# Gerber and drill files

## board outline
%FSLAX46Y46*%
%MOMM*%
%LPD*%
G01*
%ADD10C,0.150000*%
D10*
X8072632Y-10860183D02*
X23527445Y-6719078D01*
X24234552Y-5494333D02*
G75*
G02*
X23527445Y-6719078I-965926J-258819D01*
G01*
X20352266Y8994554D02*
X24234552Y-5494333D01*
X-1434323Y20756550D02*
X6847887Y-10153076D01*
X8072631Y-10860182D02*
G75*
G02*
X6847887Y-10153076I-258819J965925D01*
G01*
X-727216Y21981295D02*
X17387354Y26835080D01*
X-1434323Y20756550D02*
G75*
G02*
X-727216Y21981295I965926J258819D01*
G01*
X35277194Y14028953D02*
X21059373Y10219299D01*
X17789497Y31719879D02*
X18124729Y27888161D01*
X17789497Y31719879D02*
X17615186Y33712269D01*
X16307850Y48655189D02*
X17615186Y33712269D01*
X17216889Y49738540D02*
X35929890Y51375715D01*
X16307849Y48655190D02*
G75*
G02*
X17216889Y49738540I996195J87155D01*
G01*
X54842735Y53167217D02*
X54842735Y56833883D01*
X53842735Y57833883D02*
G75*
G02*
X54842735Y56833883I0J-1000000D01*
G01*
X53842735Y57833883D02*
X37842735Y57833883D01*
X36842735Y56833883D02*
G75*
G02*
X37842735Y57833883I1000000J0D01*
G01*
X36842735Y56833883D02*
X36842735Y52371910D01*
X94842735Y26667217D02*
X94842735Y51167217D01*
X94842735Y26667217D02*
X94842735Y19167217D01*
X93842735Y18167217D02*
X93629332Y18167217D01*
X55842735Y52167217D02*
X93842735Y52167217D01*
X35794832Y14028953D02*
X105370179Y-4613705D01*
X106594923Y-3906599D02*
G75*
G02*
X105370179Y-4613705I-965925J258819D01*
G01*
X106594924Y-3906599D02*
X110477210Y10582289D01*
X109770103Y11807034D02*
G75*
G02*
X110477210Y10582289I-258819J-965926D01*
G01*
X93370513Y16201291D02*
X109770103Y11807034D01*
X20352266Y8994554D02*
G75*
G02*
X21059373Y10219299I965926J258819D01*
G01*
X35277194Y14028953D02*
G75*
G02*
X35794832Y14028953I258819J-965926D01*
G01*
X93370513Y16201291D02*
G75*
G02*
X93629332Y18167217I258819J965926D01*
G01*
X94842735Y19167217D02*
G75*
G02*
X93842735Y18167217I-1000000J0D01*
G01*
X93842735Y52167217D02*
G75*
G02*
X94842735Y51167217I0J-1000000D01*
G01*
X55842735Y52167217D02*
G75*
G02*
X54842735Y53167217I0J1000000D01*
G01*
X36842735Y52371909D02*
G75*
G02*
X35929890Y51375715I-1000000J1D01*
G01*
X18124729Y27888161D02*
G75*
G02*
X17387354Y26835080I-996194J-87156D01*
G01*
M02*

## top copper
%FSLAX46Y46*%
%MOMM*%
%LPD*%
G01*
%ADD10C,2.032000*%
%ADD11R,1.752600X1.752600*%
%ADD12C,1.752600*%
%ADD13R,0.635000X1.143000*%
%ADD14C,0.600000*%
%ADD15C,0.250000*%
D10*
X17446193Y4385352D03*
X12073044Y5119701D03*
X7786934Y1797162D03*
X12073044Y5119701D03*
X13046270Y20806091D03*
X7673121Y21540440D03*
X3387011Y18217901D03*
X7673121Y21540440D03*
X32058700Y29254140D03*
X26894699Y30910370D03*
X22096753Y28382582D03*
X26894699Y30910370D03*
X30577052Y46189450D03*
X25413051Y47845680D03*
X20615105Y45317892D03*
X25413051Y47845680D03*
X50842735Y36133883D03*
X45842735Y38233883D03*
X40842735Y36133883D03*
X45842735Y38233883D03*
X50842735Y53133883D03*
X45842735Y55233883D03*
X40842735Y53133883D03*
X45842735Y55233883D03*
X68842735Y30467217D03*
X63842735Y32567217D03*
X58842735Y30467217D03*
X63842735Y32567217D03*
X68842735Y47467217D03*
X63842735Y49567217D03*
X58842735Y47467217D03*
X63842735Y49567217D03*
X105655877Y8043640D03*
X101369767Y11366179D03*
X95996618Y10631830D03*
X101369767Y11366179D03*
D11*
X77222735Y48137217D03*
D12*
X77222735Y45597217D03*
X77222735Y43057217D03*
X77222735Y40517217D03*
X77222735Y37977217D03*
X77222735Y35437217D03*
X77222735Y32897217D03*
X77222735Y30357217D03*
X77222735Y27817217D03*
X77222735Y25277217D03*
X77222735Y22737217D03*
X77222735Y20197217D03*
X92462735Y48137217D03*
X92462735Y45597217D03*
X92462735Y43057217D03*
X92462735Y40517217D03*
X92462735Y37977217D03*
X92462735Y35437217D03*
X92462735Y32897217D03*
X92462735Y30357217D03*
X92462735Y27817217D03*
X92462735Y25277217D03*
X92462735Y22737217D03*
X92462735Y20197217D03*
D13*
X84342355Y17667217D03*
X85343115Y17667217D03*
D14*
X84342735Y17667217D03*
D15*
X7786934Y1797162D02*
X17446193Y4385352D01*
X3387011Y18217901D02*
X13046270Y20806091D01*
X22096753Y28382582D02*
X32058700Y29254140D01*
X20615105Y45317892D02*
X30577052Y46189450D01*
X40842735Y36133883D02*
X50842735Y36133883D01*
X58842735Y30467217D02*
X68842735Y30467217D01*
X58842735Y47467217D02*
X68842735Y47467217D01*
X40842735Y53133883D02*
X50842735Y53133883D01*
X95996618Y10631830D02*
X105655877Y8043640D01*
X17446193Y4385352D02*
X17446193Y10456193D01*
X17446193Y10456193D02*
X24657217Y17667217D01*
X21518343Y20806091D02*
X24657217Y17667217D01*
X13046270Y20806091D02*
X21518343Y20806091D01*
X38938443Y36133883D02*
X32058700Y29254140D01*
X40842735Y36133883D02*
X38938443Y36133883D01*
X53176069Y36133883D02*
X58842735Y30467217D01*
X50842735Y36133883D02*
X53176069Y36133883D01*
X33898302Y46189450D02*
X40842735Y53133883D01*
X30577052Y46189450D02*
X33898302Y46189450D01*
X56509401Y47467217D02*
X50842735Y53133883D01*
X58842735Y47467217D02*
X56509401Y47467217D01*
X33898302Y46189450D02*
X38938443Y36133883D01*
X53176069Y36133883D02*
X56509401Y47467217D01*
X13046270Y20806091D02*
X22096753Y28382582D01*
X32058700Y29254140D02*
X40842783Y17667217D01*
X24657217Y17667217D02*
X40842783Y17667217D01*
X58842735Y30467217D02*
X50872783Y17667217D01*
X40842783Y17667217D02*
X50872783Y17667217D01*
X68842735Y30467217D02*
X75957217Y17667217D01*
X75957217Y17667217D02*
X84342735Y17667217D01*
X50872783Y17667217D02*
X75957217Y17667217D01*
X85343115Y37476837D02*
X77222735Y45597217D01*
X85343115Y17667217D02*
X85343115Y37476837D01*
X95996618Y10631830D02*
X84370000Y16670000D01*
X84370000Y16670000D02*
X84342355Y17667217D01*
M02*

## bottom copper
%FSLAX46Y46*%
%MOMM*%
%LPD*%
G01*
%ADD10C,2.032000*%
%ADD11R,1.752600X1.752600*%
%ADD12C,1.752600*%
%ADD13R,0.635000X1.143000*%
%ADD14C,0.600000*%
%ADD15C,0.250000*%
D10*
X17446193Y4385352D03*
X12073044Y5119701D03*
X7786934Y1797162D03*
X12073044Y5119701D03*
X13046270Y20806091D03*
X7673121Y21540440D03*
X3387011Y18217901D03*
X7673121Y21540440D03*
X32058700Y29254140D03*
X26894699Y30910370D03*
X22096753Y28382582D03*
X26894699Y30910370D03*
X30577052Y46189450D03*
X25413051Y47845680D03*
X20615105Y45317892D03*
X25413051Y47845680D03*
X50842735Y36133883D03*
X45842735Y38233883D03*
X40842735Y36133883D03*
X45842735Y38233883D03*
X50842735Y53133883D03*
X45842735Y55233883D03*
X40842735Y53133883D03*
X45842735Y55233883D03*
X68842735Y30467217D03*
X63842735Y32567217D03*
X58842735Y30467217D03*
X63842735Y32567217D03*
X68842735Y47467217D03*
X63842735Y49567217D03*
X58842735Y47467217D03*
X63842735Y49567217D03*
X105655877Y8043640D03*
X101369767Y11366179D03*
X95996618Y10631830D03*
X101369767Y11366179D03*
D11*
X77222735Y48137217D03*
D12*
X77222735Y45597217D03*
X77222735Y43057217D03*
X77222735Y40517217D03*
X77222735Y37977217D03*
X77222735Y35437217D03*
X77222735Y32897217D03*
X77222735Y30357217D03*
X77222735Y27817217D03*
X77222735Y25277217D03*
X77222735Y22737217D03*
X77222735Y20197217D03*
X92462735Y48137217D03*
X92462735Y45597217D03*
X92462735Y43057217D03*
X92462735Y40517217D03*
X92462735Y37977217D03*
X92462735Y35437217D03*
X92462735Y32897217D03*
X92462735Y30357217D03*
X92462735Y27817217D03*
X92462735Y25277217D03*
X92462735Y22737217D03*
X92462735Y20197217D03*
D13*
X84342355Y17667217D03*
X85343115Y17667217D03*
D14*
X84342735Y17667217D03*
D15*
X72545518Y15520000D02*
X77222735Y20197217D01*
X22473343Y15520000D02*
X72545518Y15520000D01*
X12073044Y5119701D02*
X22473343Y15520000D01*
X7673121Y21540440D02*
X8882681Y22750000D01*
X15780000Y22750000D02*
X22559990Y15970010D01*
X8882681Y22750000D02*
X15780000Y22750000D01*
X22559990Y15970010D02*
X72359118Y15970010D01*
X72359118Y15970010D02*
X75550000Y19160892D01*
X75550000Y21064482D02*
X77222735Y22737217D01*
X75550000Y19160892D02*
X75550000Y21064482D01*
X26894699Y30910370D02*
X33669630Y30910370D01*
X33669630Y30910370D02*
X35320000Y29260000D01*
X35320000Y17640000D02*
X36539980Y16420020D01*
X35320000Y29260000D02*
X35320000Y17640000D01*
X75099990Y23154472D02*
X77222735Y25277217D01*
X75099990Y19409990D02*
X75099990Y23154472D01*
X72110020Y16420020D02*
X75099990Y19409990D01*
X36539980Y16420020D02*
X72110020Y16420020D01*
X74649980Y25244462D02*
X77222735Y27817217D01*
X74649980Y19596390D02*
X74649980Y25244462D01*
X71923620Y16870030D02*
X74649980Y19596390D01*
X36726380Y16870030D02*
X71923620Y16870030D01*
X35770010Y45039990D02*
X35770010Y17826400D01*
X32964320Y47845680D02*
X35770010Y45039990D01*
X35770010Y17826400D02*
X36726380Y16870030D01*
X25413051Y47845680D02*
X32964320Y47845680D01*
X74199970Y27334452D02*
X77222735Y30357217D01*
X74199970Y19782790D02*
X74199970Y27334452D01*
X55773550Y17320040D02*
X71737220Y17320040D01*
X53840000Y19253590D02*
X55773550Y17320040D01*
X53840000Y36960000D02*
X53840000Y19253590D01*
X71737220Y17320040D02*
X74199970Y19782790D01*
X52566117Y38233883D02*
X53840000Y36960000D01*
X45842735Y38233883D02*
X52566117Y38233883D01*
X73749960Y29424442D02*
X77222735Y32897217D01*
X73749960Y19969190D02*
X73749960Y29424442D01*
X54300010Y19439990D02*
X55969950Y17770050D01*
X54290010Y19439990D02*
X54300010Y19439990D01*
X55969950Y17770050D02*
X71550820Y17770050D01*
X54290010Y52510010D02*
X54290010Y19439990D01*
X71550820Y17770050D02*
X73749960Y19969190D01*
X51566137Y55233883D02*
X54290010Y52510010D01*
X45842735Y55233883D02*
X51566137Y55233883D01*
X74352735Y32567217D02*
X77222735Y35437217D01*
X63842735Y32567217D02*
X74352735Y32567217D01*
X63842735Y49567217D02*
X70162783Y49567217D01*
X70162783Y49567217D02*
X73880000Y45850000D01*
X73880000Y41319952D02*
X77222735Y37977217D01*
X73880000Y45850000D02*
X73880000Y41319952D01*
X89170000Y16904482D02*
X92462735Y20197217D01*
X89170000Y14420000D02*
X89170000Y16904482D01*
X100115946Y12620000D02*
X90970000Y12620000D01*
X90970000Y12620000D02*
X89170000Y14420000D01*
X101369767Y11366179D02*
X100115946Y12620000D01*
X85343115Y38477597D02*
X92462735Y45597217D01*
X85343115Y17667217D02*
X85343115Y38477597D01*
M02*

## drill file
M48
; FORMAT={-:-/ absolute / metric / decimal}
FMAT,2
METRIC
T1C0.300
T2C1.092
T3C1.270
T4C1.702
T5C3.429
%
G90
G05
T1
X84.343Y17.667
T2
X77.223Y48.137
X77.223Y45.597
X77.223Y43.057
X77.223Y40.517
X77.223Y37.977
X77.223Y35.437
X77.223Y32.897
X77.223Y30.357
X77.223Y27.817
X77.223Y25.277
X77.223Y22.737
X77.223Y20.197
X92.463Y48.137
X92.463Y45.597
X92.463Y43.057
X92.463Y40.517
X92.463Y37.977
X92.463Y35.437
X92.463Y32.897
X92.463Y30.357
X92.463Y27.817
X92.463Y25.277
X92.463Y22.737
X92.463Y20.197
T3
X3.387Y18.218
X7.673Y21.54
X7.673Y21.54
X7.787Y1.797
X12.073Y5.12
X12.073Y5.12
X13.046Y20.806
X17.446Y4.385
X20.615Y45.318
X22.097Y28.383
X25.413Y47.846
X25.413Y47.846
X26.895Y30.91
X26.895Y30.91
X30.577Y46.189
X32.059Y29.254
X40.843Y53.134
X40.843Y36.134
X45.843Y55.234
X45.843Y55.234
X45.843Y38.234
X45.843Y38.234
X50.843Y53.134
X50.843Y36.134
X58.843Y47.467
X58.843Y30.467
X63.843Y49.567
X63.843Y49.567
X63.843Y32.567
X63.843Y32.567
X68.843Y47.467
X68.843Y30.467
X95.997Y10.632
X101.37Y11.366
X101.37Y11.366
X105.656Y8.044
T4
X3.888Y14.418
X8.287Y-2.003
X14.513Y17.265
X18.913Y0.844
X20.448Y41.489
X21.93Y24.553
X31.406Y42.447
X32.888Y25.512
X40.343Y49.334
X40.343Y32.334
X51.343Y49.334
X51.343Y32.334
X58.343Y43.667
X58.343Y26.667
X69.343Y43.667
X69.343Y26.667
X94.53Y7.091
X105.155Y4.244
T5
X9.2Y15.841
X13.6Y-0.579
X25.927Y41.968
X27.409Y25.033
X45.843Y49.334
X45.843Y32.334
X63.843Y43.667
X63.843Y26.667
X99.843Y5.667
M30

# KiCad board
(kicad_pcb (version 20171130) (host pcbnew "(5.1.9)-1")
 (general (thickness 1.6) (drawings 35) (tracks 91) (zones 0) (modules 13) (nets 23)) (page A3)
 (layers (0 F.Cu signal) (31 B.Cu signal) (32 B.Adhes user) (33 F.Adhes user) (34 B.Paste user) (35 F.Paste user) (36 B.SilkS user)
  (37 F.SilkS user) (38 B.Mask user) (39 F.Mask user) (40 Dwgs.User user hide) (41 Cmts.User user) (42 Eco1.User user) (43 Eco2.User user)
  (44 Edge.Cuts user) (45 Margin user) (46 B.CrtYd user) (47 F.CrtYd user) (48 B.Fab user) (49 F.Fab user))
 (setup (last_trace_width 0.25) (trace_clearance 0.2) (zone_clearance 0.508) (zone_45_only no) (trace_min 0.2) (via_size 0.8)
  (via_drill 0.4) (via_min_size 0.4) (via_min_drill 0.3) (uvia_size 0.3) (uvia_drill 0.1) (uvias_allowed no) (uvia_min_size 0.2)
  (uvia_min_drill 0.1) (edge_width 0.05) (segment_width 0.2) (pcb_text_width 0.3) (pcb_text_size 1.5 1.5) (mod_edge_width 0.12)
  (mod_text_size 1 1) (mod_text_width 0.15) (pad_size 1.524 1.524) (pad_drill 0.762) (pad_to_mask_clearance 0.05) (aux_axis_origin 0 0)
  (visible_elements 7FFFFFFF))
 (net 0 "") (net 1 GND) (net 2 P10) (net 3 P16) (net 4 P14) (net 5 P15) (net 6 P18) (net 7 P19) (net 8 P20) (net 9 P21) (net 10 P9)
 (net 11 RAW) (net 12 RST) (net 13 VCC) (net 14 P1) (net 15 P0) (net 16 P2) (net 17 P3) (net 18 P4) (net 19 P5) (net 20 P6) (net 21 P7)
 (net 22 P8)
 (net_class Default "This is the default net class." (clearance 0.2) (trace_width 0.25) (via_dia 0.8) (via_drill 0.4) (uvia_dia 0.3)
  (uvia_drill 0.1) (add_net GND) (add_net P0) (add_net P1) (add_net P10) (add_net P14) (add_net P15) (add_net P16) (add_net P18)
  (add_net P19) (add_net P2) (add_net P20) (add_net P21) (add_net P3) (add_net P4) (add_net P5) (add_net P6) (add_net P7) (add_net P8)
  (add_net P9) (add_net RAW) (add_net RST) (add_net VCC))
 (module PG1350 (layer F.Cu) (at 13.600076 0.579261 15)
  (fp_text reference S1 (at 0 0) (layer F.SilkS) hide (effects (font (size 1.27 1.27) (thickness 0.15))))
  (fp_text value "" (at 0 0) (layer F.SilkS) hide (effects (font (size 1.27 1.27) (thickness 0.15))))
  (pad "" np_thru_hole circle (at 0 0) (size 3.429 3.429) (drill 3.429) (layers *.Cu *.Mask))
  (pad "" np_thru_hole circle (at 5.5 0) (size 1.7018 1.7018) (drill 1.7018) (layers *.Cu *.Mask))
  (pad "" np_thru_hole circle (at -5.5 0) (size 1.7018 1.7018) (drill 1.7018) (layers *.Cu *.Mask))
  (pad 1 thru_hole circle (at 5 -3.8) (size 2.032 2.032) (drill 1.27) (layers *.Cu *.Mask) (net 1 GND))
  (pad 2 thru_hole circle (at 0 -5.9) (size 2.032 2.032) (drill 1.27) (layers *.Cu *.Mask) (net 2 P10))
  (pad 1 thru_hole circle (at -5 -3.8) (size 2.032 2.032) (drill 1.27) (layers *.Cu *.Mask) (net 1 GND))
  (pad 2 thru_hole circle (at 0 -5.9) (size 2.032 2.032) (drill 1.27) (layers *.Cu *.Mask) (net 2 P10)))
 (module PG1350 (layer F.Cu) (at 9.200153 -15.841478 15)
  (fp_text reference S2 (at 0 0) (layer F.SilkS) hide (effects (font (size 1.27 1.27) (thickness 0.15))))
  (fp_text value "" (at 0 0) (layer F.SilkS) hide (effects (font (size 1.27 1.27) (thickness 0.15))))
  (pad "" np_thru_hole circle (at 0 0) (size 3.429 3.429) (drill 3.429) (layers *.Cu *.Mask))
  (pad "" np_thru_hole circle (at 5.5 0) (size 1.7018 1.7018) (drill 1.7018) (layers *.Cu *.Mask))
  (pad "" np_thru_hole circle (at -5.5 0) (size 1.7018 1.7018) (drill 1.7018) (layers *.Cu *.Mask))
  (pad 1 thru_hole circle (at 5 -3.8) (size 2.032 2.032) (drill 1.27) (layers *.Cu *.Mask) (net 1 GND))
  (pad 2 thru_hole circle (at 0 -5.9) (size 2.032 2.032) (drill 1.27) (layers *.Cu *.Mask) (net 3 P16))
  (pad 1 thru_hole circle (at -5 -3.8) (size 2.032 2.032) (drill 1.27) (layers *.Cu *.Mask) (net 1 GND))
  (pad 2 thru_hole circle (at 0 -5.9) (size 2.032 2.032) (drill 1.27) (layers *.Cu *.Mask) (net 3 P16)))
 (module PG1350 (layer F.Cu) (at 27.408918 -25.032821 5)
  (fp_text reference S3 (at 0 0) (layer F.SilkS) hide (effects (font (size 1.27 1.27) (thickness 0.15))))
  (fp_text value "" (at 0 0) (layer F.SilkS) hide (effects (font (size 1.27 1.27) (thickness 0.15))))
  (pad "" np_thru_hole circle (at 0 0) (size 3.429 3.429) (drill 3.429) (layers *.Cu *.Mask))
  (pad "" np_thru_hole circle (at 5.5 0) (size 1.7018 1.7018) (drill 1.7018) (layers *.Cu *.Mask))
  (pad "" np_thru_hole circle (at -5.5 0) (size 1.7018 1.7018) (drill 1.7018) (layers *.Cu *.Mask))
  (pad 1 thru_hole circle (at 5 -3.8) (size 2.032 2.032) (drill 1.27) (layers *.Cu *.Mask) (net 1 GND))
  (pad 2 thru_hole circle (at 0 -5.9) (size 2.032 2.032) (drill 1.27) (layers *.Cu *.Mask) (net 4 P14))
  (pad 1 thru_hole circle (at -5 -3.8) (size 2.032 2.032) (drill 1.27) (layers *.Cu *.Mask) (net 1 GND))
  (pad 2 thru_hole circle (at 0 -5.9) (size 2.032 2.032) (drill 1.27) (layers *.Cu *.Mask) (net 4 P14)))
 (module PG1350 (layer F.Cu) (at 25.92727 -41.968131 5)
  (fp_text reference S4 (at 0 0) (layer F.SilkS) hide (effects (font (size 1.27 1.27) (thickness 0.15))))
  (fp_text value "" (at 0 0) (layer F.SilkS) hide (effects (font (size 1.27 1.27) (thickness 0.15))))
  (pad "" np_thru_hole circle (at 0 0) (size 3.429 3.429) (drill 3.429) (layers *.Cu *.Mask))
  (pad "" np_thru_hole circle (at 5.5 0) (size 1.7018 1.7018) (drill 1.7018) (layers *.Cu *.Mask))
  (pad "" np_thru_hole circle (at -5.5 0) (size 1.7018 1.7018) (drill 1.7018) (layers *.Cu *.Mask))
  (pad 1 thru_hole circle (at 5 -3.8) (size 2.032 2.032) (drill 1.27) (layers *.Cu *.Mask) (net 1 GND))
  (pad 2 thru_hole circle (at 0 -5.9) (size 2.032 2.032) (drill 1.27) (layers *.Cu *.Mask) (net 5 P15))
  (pad 1 thru_hole circle (at -5 -3.8) (size 2.032 2.032) (drill 1.27) (layers *.Cu *.Mask) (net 1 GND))
  (pad 2 thru_hole circle (at 0 -5.9) (size 2.032 2.032) (drill 1.27) (layers *.Cu *.Mask) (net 5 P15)))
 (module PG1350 (layer F.Cu) (at 45.842735 -32.333883)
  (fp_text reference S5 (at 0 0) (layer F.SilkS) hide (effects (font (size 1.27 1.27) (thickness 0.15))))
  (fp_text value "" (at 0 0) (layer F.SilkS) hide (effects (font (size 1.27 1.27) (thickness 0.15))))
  (pad "" np_thru_hole circle (at 0 0) (size 3.429 3.429) (drill 3.429) (layers *.Cu *.Mask))
  (pad "" np_thru_hole circle (at 5.5 0) (size 1.7018 1.7018) (drill 1.7018) (layers *.Cu *.Mask))
  (pad "" np_thru_hole circle (at -5.5 0) (size 1.7018 1.7018) (drill 1.7018) (layers *.Cu *.Mask))
  (pad 1 thru_hole circle (at 5 -3.8) (size 2.032 2.032) (drill 1.27) (layers *.Cu *.Mask) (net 1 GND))
  (pad 2 thru_hole circle (at 0 -5.9) (size 2.032 2.032) (drill 1.27) (layers *.Cu *.Mask) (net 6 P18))
  (pad 1 thru_hole circle (at -5 -3.8) (size 2.032 2.032) (drill 1.27) (layers *.Cu *.Mask) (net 1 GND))
  (pad 2 thru_hole circle (at 0 -5.9) (size 2.032 2.032) (drill 1.27) (layers *.Cu *.Mask) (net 6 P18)))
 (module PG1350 (layer F.Cu) (at 45.842735 -49.333883)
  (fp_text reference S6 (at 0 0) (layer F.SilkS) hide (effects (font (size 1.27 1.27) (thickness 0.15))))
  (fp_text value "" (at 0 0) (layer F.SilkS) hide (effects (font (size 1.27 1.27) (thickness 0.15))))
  (pad "" np_thru_hole circle (at 0 0) (size 3.429 3.429) (drill 3.429) (layers *.Cu *.Mask))
  (pad "" np_thru_hole circle (at 5.5 0) (size 1.7018 1.7018) (drill 1.7018) (layers *.Cu *.Mask))
  (pad "" np_thru_hole circle (at -5.5 0) (size 1.7018 1.7018) (drill 1.7018) (layers *.Cu *.Mask))
  (pad 1 thru_hole circle (at 5 -3.8) (size 2.032 2.032) (drill 1.27) (layers *.Cu *.Mask) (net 1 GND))
  (pad 2 thru_hole circle (at 0 -5.9) (size 2.032 2.032) (drill 1.27) (layers *.Cu *.Mask) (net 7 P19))
  (pad 1 thru_hole circle (at -5 -3.8) (size 2.032 2.032) (drill 1.27) (layers *.Cu *.Mask) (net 1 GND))
  (pad 2 thru_hole circle (at 0 -5.9) (size 2.032 2.032) (drill 1.27) (layers *.Cu *.Mask) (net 7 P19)))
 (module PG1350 (layer F.Cu) (at 63.842735 -26.667217)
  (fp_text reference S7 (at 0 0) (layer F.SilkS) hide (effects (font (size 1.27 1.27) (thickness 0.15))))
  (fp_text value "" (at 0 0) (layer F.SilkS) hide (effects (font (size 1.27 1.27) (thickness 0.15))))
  (pad "" np_thru_hole circle (at 0 0) (size 3.429 3.429) (drill 3.429) (layers *.Cu *.Mask))
  (pad "" np_thru_hole circle (at 5.5 0) (size 1.7018 1.7018) (drill 1.7018) (layers *.Cu *.Mask))
  (pad "" np_thru_hole circle (at -5.5 0) (size 1.7018 1.7018) (drill 1.7018) (layers *.Cu *.Mask))
  (pad 1 thru_hole circle (at 5 -3.8) (size 2.032 2.032) (drill 1.27) (layers *.Cu *.Mask) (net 1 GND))
  (pad 2 thru_hole circle (at 0 -5.9) (size 2.032 2.032) (drill 1.27) (layers *.Cu *.Mask) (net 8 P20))
  (pad 1 thru_hole circle (at -5 -3.8) (size 2.032 2.032) (drill 1.27) (layers *.Cu *.Mask) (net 1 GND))
  (pad 2 thru_hole circle (at 0 -5.9) (size 2.032 2.032) (drill 1.27) (layers *.Cu *.Mask) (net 8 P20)))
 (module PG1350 (layer F.Cu) (at 63.842735 -43.667217)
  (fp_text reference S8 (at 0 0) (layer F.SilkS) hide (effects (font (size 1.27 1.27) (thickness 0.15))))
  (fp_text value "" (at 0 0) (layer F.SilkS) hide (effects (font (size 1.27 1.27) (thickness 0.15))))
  (pad "" np_thru_hole circle (at 0 0) (size 3.429 3.429) (drill 3.429) (layers *.Cu *.Mask))
  (pad "" np_thru_hole circle (at 5.5 0) (size 1.7018 1.7018) (drill 1.7018) (layers *.Cu *.Mask))
  (pad "" np_thru_hole circle (at -5.5 0) (size 1.7018 1.7018) (drill 1.7018) (layers *.Cu *.Mask))
  (pad 1 thru_hole circle (at 5 -3.8) (size 2.032 2.032) (drill 1.27) (layers *.Cu *.Mask) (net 1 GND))
  (pad 2 thru_hole circle (at 0 -5.9) (size 2.032 2.032) (drill 1.27) (layers *.Cu *.Mask) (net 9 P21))
  (pad 1 thru_hole circle (at -5 -3.8) (size 2.032 2.032) (drill 1.27) (layers *.Cu *.Mask) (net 1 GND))
  (pad 2 thru_hole circle (at 0 -5.9) (size 2.032 2.032) (drill 1.27) (layers *.Cu *.Mask) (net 9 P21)))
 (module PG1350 (layer F.Cu) (at 99.842735 -5.667217 345)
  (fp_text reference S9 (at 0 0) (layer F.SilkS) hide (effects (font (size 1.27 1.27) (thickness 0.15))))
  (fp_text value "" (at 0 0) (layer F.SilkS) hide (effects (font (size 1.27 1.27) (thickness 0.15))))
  (pad "" np_thru_hole circle (at 0 0) (size 3.429 3.429) (drill 3.429) (layers *.Cu *.Mask))
  (pad "" np_thru_hole circle (at 5.5 0) (size 1.7018 1.7018) (drill 1.7018) (layers *.Cu *.Mask))
  (pad "" np_thru_hole circle (at -5.5 0) (size 1.7018 1.7018) (drill 1.7018) (layers *.Cu *.Mask))
  (pad 1 thru_hole circle (at 5 -3.8) (size 2.032 2.032) (drill 1.27) (layers *.Cu *.Mask) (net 1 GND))
  (pad 2 thru_hole circle (at 0 -5.9) (size 2.032 2.032) (drill 1.27) (layers *.Cu *.Mask) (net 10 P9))
  (pad 1 thru_hole circle (at -5 -3.8) (size 2.032 2.032) (drill 1.27) (layers *.Cu *.Mask) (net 1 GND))
  (pad 2 thru_hole circle (at 0 -5.9) (size 2.032 2.032) (drill 1.27) (layers *.Cu *.Mask) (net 10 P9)))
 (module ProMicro (layer F.Cu) (at 84.842735 -34.167217 270)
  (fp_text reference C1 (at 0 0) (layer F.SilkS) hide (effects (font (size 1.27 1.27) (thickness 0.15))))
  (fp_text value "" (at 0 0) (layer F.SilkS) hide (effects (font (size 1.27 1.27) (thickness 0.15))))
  (pad 1 thru_hole rect (at -13.97 7.62 270) (size 1.7526 1.7526) (drill 1.0922) (layers *.Cu *.SilkS *.Mask) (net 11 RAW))
  (pad 2 thru_hole circle (at -11.43 7.62) (size 1.7526 1.7526) (drill 1.0922) (layers *.Cu *.SilkS *.Mask) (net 1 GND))
  (pad 3 thru_hole circle (at -8.89 7.62) (size 1.7526 1.7526) (drill 1.0922) (layers *.Cu *.SilkS *.Mask) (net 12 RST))
  (pad 4 thru_hole circle (at -6.35 7.62) (size 1.7526 1.7526) (drill 1.0922) (layers *.Cu *.SilkS *.Mask) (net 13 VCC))
  (pad 5 thru_hole circle (at -3.81 7.62) (size 1.7526 1.7526) (drill 1.0922) (layers *.Cu *.SilkS *.Mask) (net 9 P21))
  (pad 6 thru_hole circle (at -1.27 7.62) (size 1.7526 1.7526) (drill 1.0922) (layers *.Cu *.SilkS *.Mask) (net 8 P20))
  (pad 7 thru_hole circle (at 1.27 7.62) (size 1.7526 1.7526) (drill 1.0922) (layers *.Cu *.SilkS *.Mask) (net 7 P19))
  (pad 8 thru_hole circle (at 3.81 7.62) (size 1.7526 1.7526) (drill 1.0922) (layers *.Cu *.SilkS *.Mask) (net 6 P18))
  (pad 9 thru_hole circle (at 6.35 7.62) (size 1.7526 1.7526) (drill 1.0922) (layers *.Cu *.SilkS *.Mask) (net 5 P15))
  (pad 10 thru_hole circle (at 8.89 7.62) (size 1.7526 1.7526) (drill 1.0922) (layers *.Cu *.SilkS *.Mask) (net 4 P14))
  (pad 11 thru_hole circle (at 11.43 7.62) (size 1.7526 1.7526) (drill 1.0922) (layers *.Cu *.SilkS *.Mask) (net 3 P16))
  (pad 12 thru_hole circle (at 13.97 7.62) (size 1.7526 1.7526) (drill 1.0922) (layers *.Cu *.SilkS *.Mask) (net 2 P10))
  (pad 13 thru_hole circle (at -13.97 -7.62) (size 1.7526 1.7526) (drill 1.0922) (layers *.Cu *.SilkS *.Mask) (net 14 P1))
  (pad 14 thru_hole circle (at -11.43 -7.62) (size 1.7526 1.7526) (drill 1.0922) (layers *.Cu *.SilkS *.Mask) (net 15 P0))
  (pad 15 thru_hole circle (at -8.89 -7.62) (size 1.7526 1.7526) (drill 1.0922) (layers *.Cu *.SilkS *.Mask) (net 1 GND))
  (pad 16 thru_hole circle (at -6.35 -7.62) (size 1.7526 1.7526) (drill 1.0922) (layers *.Cu *.SilkS *.Mask) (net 1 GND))
  (pad 17 thru_hole circle (at -3.81 -7.62) (size 1.7526 1.7526) (drill 1.0922) (layers *.Cu *.SilkS *.Mask) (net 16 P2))
  (pad 18 thru_hole circle (at -1.27 -7.62) (size 1.7526 1.7526) (drill 1.0922) (layers *.Cu *.SilkS *.Mask) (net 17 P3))
  (pad 19 thru_hole circle (at 1.27 -7.62) (size 1.7526 1.7526) (drill 1.0922) (layers *.Cu *.SilkS *.Mask) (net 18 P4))
  (pad 20 thru_hole circle (at 3.81 -7.62) (size 1.7526 1.7526) (drill 1.0922) (layers *.Cu *.SilkS *.Mask) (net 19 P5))
  (pad 21 thru_hole circle (at 6.35 -7.62) (size 1.7526 1.7526) (drill 1.0922) (layers *.Cu *.SilkS *.Mask) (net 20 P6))
  (pad 22 thru_hole circle (at 8.89 -7.62) (size 1.7526 1.7526) (drill 1.0922) (layers *.Cu *.SilkS *.Mask) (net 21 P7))
  (pad 23 thru_hole circle (at 11.43 -7.62) (size 1.7526 1.7526) (drill 1.0922) (layers *.Cu *.SilkS *.Mask) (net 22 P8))
  (pad 24 thru_hole circle (at 13.97 -7.62) (size 1.7526 1.7526) (drill 1.0922) (layers *.Cu *.SilkS *.Mask) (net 10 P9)))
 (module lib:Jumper (layer F.Cu) (at 84.842735 -17.667217)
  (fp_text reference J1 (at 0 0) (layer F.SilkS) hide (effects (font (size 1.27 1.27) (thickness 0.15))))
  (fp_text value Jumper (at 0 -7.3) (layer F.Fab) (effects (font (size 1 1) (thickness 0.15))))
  (pad 1 smd rect (at -0.50038 0) (size 0.635 1.143) (layers F.Cu F.Paste F.Mask) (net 1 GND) (clearance 0.1905))
  (pad 2 smd rect (at 0.50038 0) (size 0.635 1.143) (layers F.Cu F.Paste F.Mask) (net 1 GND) (clearance 0.1905)))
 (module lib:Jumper (layer F.Cu) (at 84.842735 -17.667217)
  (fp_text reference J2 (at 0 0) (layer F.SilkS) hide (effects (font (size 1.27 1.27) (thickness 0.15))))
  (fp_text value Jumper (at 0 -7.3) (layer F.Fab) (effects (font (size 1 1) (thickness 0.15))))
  (pad 1 smd rect (at -0.50038 0) (size 0.635 1.143) (layers B.Cu B.Paste B.Mask) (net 1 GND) (clearance 0.1905))
  (pad 2 smd rect (at 0.50038 0) (size 0.635 1.143) (layers B.Cu B.Paste B.Mask) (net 15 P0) (clearance 0.1905)))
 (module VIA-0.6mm (layer F.Cu) (at 84.342735 -17.667217)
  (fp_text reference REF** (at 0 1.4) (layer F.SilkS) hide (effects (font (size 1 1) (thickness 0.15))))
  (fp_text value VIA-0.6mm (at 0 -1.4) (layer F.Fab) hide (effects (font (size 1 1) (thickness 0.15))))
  (pad 1 thru_hole circle (at 0 0) (size 0.6 0.6) (drill 0.3) (layers *.Cu) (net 1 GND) (zone_connect 2)))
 (gr_line (start 8.072632 10.860183) (end 23.527445 6.719078) (angle 90) (layer Edge.Cuts) (width 0.15))
 (gr_arc (start 23.268626 5.753152) (end 23.527445 6.719078) (angle -90) (layer Edge.Cuts) (width 0.15))
 (gr_line (start 20.352266 -8.994554) (end 24.234552 5.494333) (angle 90) (layer Edge.Cuts) (width 0.15))
 (gr_line (start -1.434323 -20.75655) (end 6.847887 10.153076) (angle 90) (layer Edge.Cuts) (width 0.15))
 (gr_arc (start 7.813812 9.894257) (end 6.847887 10.153076) (angle -90) (layer Edge.Cuts) (width 0.15))
 (gr_line (start -0.727216 -21.981295) (end 17.387354 -26.83508) (angle 90) (layer Edge.Cuts) (width 0.15))
 (gr_arc (start -0.468397 -21.015369) (end -0.727216 -21.981295) (angle -90) (layer Edge.Cuts) (width 0.15))
 (gr_line (start 35.277194 -14.028953) (end 21.059373 -10.219299) (angle 90) (layer Edge.Cuts) (width 0.15))
 (gr_line (start 17.789497 -31.719879) (end 18.124729 -27.888161) (angle 90) (layer Edge.Cuts) (width 0.15))
 (gr_line (start 17.789497 -31.719879) (end 17.615186 -33.712269) (angle 90) (layer Edge.Cuts) (width 0.15))
 (gr_line (start 16.30785 -48.655189) (end 17.615186 -33.712269) (angle 90) (layer Edge.Cuts) (width 0.15))
 (gr_line (start 17.216889 -49.73854) (end 35.92989 -51.375715) (angle 90) (layer Edge.Cuts) (width 0.15))
 (gr_arc (start 17.304044 -48.742345) (end 17.216889 -49.73854) (angle -90) (layer Edge.Cuts) (width 0.15))
 (gr_line (start 54.842735 -53.167217) (end 54.842735 -56.833883) (angle 90) (layer Edge.Cuts) (width 0.15))
 (gr_arc (start 53.842735 -56.833883) (end 54.842735 -56.833883) (angle -90) (layer Edge.Cuts) (width 0.15))
 (gr_line (start 53.842735 -57.833883) (end 37.842735 -57.833883) (angle 90) (layer Edge.Cuts) (width 0.15))
 (gr_arc (start 37.842735 -56.833883) (end 37.842735 -57.833883) (angle -90) (layer Edge.Cuts) (width 0.15))
 (gr_line (start 36.842735 -56.833883) (end 36.842735 -52.37191) (angle 90) (layer Edge.Cuts) (width 0.15))
 (gr_line (start 94.842735 -26.667217) (end 94.842735 -51.167217) (angle 90) (layer Edge.Cuts) (width 0.15))
 (gr_line (start 94.842735 -26.667217) (end 94.842735 -19.167217) (angle 90) (layer Edge.Cuts) (width 0.15))
 (gr_line (start 93.842735 -18.167217) (end 93.629332 -18.167217) (angle 90) (layer Edge.Cuts) (width 0.15))
 (gr_line (start 55.842735 -52.167217) (end 93.842735 -52.167217) (angle 90) (layer Edge.Cuts) (width 0.15))
 (gr_line (start 35.794832 -14.028953) (end 105.370179 4.613705) (angle 90) (layer Edge.Cuts) (width 0.15))
 (gr_arc (start 105.628998 3.64778) (end 105.370179 4.613705) (angle -90) (layer Edge.Cuts) (width 0.15))
 (gr_line (start 106.594924 3.906599) (end 110.47721 -10.582289) (angle 90) (layer Edge.Cuts) (width 0.15))
 (gr_arc (start 109.511284 -10.841108) (end 110.47721 -10.582289) (angle -90) (layer Edge.Cuts) (width 0.15))
 (gr_line (start 93.370513 -16.201291) (end 109.770103 -11.807034) (angle 90) (layer Edge.Cuts) (width 0.15))
 (gr_arc (start 21.318192 -9.253373) (end 21.059373 -10.219299) (angle -90) (layer Edge.Cuts) (width 0.15))
 (gr_arc (start 35.536013 -13.063027) (end 35.794832 -14.028953) (angle -29.99999579) (layer Edge.Cuts) (width 0.15))
 (gr_arc (start 93.629332 -17.167217) (end 93.629332 -18.167217) (angle -165.0000021) (layer Edge.Cuts) (width 0.15))
 (gr_arc (start 93.842735 -19.167217) (end 93.842735 -18.167217) (angle -90) (layer Edge.Cuts) (width 0.15))
 (gr_arc (start 93.842735 -51.167217) (end 94.842735 -51.167217) (angle -90) (layer Edge.Cuts) (width 0.15))
 (gr_arc (start 55.842735 -53.167217) (end 54.842735 -53.167217) (angle -90) (layer Edge.Cuts) (width 0.15))
 (gr_arc (start 35.842735 -52.37191) (end 35.92989 -51.375715) (angle -85.00000245) (layer Edge.Cuts) (width 0.15))
 (gr_arc (start 17.128535 -27.801005) (end 17.387354 -26.83508) (angle -79.99999966) (layer Edge.Cuts) (width 0.15))
 (segment (start 7.786934 -1.797162) (end 17.446193 -4.385352) (width 0.25) (layer F.Cu) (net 1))
 (segment (start 3.387011 -18.217901) (end 13.04627 -20.806091) (width 0.25) (layer F.Cu) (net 1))
 (segment (start 22.096753 -28.382582) (end 32.0587 -29.25414) (width 0.25) (layer F.Cu) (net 1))
 (segment (start 20.615105 -45.317892) (end 30.577052 -46.18945) (width 0.25) (layer F.Cu) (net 1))
 (segment (start 40.842735 -36.133883) (end 50.842735 -36.133883) (width 0.25) (layer F.Cu) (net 1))
 (segment (start 58.842735 -30.467217) (end 68.842735 -30.467217) (width 0.25) (layer F.Cu) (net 1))
 (segment (start 58.842735 -47.467217) (end 68.842735 -47.467217) (width 0.25) (layer F.Cu) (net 1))
 (segment (start 40.842735 -53.133883) (end 50.842735 -53.133883) (width 0.25) (layer F.Cu) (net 1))
 (segment (start 95.996618 -10.63183) (end 105.655877 -8.04364) (width 0.25) (layer F.Cu) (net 1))
 (segment (start 17.446193 -4.385352) (end 17.446193 -10.456193) (width 0.25) (layer F.Cu) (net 1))
 (segment (start 17.446193 -10.456193) (end 24.657217 -17.667217) (width 0.25) (layer F.Cu) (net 1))
 (segment (start 21.518343 -20.806091) (end 24.657217 -17.667217) (width 0.25) (layer F.Cu) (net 1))
 (segment (start 13.04627 -20.806091) (end 21.518343 -20.806091) (width 0.25) (layer F.Cu) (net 1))
 (segment (start 38.938443 -36.133883) (end 32.0587 -29.25414) (width 0.25) (layer F.Cu) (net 1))
 (segment (start 40.842735 -36.133883) (end 38.938443 -36.133883) (width 0.25) (layer F.Cu) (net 1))
 (segment (start 53.176069 -36.133883) (end 58.842735 -30.467217) (width 0.25) (layer F.Cu) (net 1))
 (segment (start 50.842735 -36.133883) (end 53.176069 -36.133883) (width 0.25) (layer F.Cu) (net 1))
 (segment (start 33.898302 -46.18945) (end 40.842735 -53.133883) (width 0.25) (layer F.Cu) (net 1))
 (segment (start 30.577052 -46.18945) (end 33.898302 -46.18945) (width 0.25) (layer F.Cu) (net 1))
 (segment (start 56.509401 -47.467217) (end 50.842735 -53.133883) (width 0.25) (layer F.Cu) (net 1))
 (segment (start 58.842735 -47.467217) (end 56.509401 -47.467217) (width 0.25) (layer F.Cu) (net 1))
 (segment (start 33.898302 -46.18945) (end 38.938443 -36.133883) (width 0.25) (layer F.Cu) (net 1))
 (segment (start 53.176069 -36.133883) (end 56.509401 -47.467217) (width 0.25) (layer F.Cu) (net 1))
 (segment (start 13.04627 -20.806091) (end 22.096753 -28.382582) (width 0.25) (layer F.Cu) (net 1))
 (segment (start 32.0587 -29.25414) (end 40.842783 -17.667217) (width 0.25) (layer F.Cu) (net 1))
 (segment (start 24.657217 -17.667217) (end 40.842783 -17.667217) (width 0.25) (layer F.Cu) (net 1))
 (segment (start 58.842735 -30.467217) (end 50.872783 -17.667217) (width 0.25) (layer F.Cu) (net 1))
 (segment (start 40.842783 -17.667217) (end 50.872783 -17.667217) (width 0.25) (layer F.Cu) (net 1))
 (segment (start 68.842735 -30.467217) (end 75.957217 -17.667217) (width 0.25) (layer F.Cu) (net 1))
 (segment (start 75.957217 -17.667217) (end 84.342735 -17.667217) (width 0.25) (layer F.Cu) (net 1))
 (segment (start 50.872783 -17.667217) (end 75.957217 -17.667217) (width 0.25) (layer F.Cu) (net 1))
 (segment (start 85.343115 -37.476837) (end 77.222735 -45.597217) (width 0.25) (layer F.Cu) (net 1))
 (segment (start 85.343115 -17.667217) (end 85.343115 -37.476837) (width 0.25) (layer F.Cu) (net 1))
 (segment (start 95.996618 -10.63183) (end 84.37 -16.67) (width 0.25) (layer F.Cu) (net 1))
 (segment (start 84.37 -16.67) (end 84.342355 -17.667217) (width 0.25) (layer F.Cu) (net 1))
 (segment (start 72.545518 -15.52) (end 77.222735 -20.197217) (width 0.25) (layer B.Cu) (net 2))
 (segment (start 22.473343 -15.52) (end 72.545518 -15.52) (width 0.25) (layer B.Cu) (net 2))
 (segment (start 12.073044 -5.119701) (end 22.473343 -15.52) (width 0.25) (layer B.Cu) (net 2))
 (segment (start 7.673121 -21.54044) (end 8.882681 -22.75) (width 0.25) (layer B.Cu) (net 3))
 (segment (start 15.78 -22.75) (end 22.55999 -15.97001) (width 0.25) (layer B.Cu) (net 3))
 (segment (start 8.882681 -22.75) (end 15.78 -22.75) (width 0.25) (layer B.Cu) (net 3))
 (segment (start 22.55999 -15.97001) (end 72.359118 -15.97001) (width 0.25) (layer B.Cu) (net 3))
 (segment (start 72.359118 -15.97001) (end 75.55 -19.160892) (width 0.25) (layer B.Cu) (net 3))
 (segment (start 75.55 -21.064482) (end 77.222735 -22.737217) (width 0.25) (layer B.Cu) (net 3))
 (segment (start 75.55 -19.160892) (end 75.55 -21.064482) (width 0.25) (layer B.Cu) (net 3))
 (segment (start 26.894699 -30.91037) (end 33.66963 -30.91037) (width 0.25) (layer B.Cu) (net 4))
 (segment (start 33.66963 -30.91037) (end 35.32 -29.26) (width 0.25) (layer B.Cu) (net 4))
 (segment (start 35.32 -17.64) (end 36.53998 -16.42002) (width 0.25) (layer B.Cu) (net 4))
 (segment (start 35.32 -29.26) (end 35.32 -17.64) (width 0.25) (layer B.Cu) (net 4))
 (segment (start 75.09999 -23.154472) (end 77.222735 -25.277217) (width 0.25) (layer B.Cu) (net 4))
 (segment (start 75.09999 -19.40999) (end 75.09999 -23.154472) (width 0.25) (layer B.Cu) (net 4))
 (segment (start 72.11002 -16.42002) (end 75.09999 -19.40999) (width 0.25) (layer B.Cu) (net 4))
 (segment (start 36.53998 -16.42002) (end 72.11002 -16.42002) (width 0.25) (layer B.Cu) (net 4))
 (segment (start 74.64998 -25.244462) (end 77.222735 -27.817217) (width 0.25) (layer B.Cu) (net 5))
 (segment (start 74.64998 -19.59639) (end 74.64998 -25.244462) (width 0.25) (layer B.Cu) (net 5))
 (segment (start 71.92362 -16.87003) (end 74.64998 -19.59639) (width 0.25) (layer B.Cu) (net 5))
 (segment (start 36.72638 -16.87003) (end 71.92362 -16.87003) (width 0.25) (layer B.Cu) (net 5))
 (segment (start 35.77001 -45.03999) (end 35.77001 -17.8264) (width 0.25) (layer B.Cu) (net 5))
 (segment (start 32.96432 -47.84568) (end 35.77001 -45.03999) (width 0.25) (layer B.Cu) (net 5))
 (segment (start 35.77001 -17.8264) (end 36.72638 -16.87003) (width 0.25) (layer B.Cu) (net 5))
 (segment (start 25.413051 -47.84568) (end 32.96432 -47.84568) (width 0.25) (layer B.Cu) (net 5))
 (segment (start 74.19997 -27.334452) (end 77.222735 -30.357217) (width 0.25) (layer B.Cu) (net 6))
 (segment (start 74.19997 -19.78279) (end 74.19997 -27.334452) (width 0.25) (layer B.Cu) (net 6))
 (segment (start 55.77355 -17.32004) (end 71.73722 -17.32004) (width 0.25) (layer B.Cu) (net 6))
 (segment (start 53.84 -19.25359) (end 55.77355 -17.32004) (width 0.25) (layer B.Cu) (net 6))
 (segment (start 53.84 -36.96) (end 53.84 -19.25359) (width 0.25) (layer B.Cu) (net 6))
 (segment (start 71.73722 -17.32004) (end 74.19997 -19.78279) (width 0.25) (layer B.Cu) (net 6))
 (segment (start 52.566117 -38.233883) (end 53.84 -36.96) (width 0.25) (layer B.Cu) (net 6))
 (segment (start 45.842735 -38.233883) (end 52.566117 -38.233883) (width 0.25) (layer B.Cu) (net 6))
 (segment (start 73.74996 -29.424442) (end 77.222735 -32.897217) (width 0.25) (layer B.Cu) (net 7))
 (segment (start 73.74996 -19.96919) (end 73.74996 -29.424442) (width 0.25) (layer B.Cu) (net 7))
 (segment (start 54.30001 -19.43999) (end 55.96995 -17.77005) (width 0.25) (layer B.Cu) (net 7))
 (segment (start 54.29001 -19.43999) (end 54.30001 -19.43999) (width 0.25) (layer B.Cu) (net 7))
 (segment (start 55.96995 -17.77005) (end 71.55082 -17.77005) (width 0.25) (layer B.Cu) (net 7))
 (segment (start 54.29001 -52.51001) (end 54.29001 -19.43999) (width 0.25) (layer B.Cu) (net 7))
 (segment (start 71.55082 -17.77005) (end 73.74996 -19.96919) (width 0.25) (layer B.Cu) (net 7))
 (segment (start 51.566137 -55.233883) (end 54.29001 -52.51001) (width 0.25) (layer B.Cu) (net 7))
 (segment (start 45.842735 -55.233883) (end 51.566137 -55.233883) (width 0.25) (layer B.Cu) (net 7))
 (segment (start 74.352735 -32.567217) (end 77.222735 -35.437217) (width 0.25) (layer B.Cu) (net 8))
 (segment (start 63.842735 -32.567217) (end 74.352735 -32.567217) (width 0.25) (layer B.Cu) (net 8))
 (segment (start 63.842735 -49.567217) (end 70.162783 -49.567217) (width 0.25) (layer B.Cu) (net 9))
 (segment (start 70.162783 -49.567217) (end 73.88 -45.85) (width 0.25) (layer B.Cu) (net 9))
 (segment (start 73.88 -41.319952) (end 77.222735 -37.977217) (width 0.25) (layer B.Cu) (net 9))
 (segment (start 73.88 -45.85) (end 73.88 -41.319952) (width 0.25) (layer B.Cu) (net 9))
 (segment (start 89.17 -16.904482) (end 92.462735 -20.197217) (width 0.25) (layer B.Cu) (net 10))
 (segment (start 89.17 -14.42) (end 89.17 -16.904482) (width 0.25) (layer B.Cu) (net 10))
 (segment (start 100.115946 -12.62) (end 90.97 -12.62) (width 0.25) (layer B.Cu) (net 10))
 (segment (start 90.97 -12.62) (end 89.17 -14.42) (width 0.25) (layer B.Cu) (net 10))
 (segment (start 101.369767 -11.366179) (end 100.115946 -12.62) (width 0.25) (layer B.Cu) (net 10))
 (segment (start 85.343115 -38.477597) (end 92.462735 -45.597217) (width 0.25) (layer B.Cu) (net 15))
 (segment (start 85.343115 -17.667217) (end 85.343115 -38.477597) (width 0.25) (layer B.Cu) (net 15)))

